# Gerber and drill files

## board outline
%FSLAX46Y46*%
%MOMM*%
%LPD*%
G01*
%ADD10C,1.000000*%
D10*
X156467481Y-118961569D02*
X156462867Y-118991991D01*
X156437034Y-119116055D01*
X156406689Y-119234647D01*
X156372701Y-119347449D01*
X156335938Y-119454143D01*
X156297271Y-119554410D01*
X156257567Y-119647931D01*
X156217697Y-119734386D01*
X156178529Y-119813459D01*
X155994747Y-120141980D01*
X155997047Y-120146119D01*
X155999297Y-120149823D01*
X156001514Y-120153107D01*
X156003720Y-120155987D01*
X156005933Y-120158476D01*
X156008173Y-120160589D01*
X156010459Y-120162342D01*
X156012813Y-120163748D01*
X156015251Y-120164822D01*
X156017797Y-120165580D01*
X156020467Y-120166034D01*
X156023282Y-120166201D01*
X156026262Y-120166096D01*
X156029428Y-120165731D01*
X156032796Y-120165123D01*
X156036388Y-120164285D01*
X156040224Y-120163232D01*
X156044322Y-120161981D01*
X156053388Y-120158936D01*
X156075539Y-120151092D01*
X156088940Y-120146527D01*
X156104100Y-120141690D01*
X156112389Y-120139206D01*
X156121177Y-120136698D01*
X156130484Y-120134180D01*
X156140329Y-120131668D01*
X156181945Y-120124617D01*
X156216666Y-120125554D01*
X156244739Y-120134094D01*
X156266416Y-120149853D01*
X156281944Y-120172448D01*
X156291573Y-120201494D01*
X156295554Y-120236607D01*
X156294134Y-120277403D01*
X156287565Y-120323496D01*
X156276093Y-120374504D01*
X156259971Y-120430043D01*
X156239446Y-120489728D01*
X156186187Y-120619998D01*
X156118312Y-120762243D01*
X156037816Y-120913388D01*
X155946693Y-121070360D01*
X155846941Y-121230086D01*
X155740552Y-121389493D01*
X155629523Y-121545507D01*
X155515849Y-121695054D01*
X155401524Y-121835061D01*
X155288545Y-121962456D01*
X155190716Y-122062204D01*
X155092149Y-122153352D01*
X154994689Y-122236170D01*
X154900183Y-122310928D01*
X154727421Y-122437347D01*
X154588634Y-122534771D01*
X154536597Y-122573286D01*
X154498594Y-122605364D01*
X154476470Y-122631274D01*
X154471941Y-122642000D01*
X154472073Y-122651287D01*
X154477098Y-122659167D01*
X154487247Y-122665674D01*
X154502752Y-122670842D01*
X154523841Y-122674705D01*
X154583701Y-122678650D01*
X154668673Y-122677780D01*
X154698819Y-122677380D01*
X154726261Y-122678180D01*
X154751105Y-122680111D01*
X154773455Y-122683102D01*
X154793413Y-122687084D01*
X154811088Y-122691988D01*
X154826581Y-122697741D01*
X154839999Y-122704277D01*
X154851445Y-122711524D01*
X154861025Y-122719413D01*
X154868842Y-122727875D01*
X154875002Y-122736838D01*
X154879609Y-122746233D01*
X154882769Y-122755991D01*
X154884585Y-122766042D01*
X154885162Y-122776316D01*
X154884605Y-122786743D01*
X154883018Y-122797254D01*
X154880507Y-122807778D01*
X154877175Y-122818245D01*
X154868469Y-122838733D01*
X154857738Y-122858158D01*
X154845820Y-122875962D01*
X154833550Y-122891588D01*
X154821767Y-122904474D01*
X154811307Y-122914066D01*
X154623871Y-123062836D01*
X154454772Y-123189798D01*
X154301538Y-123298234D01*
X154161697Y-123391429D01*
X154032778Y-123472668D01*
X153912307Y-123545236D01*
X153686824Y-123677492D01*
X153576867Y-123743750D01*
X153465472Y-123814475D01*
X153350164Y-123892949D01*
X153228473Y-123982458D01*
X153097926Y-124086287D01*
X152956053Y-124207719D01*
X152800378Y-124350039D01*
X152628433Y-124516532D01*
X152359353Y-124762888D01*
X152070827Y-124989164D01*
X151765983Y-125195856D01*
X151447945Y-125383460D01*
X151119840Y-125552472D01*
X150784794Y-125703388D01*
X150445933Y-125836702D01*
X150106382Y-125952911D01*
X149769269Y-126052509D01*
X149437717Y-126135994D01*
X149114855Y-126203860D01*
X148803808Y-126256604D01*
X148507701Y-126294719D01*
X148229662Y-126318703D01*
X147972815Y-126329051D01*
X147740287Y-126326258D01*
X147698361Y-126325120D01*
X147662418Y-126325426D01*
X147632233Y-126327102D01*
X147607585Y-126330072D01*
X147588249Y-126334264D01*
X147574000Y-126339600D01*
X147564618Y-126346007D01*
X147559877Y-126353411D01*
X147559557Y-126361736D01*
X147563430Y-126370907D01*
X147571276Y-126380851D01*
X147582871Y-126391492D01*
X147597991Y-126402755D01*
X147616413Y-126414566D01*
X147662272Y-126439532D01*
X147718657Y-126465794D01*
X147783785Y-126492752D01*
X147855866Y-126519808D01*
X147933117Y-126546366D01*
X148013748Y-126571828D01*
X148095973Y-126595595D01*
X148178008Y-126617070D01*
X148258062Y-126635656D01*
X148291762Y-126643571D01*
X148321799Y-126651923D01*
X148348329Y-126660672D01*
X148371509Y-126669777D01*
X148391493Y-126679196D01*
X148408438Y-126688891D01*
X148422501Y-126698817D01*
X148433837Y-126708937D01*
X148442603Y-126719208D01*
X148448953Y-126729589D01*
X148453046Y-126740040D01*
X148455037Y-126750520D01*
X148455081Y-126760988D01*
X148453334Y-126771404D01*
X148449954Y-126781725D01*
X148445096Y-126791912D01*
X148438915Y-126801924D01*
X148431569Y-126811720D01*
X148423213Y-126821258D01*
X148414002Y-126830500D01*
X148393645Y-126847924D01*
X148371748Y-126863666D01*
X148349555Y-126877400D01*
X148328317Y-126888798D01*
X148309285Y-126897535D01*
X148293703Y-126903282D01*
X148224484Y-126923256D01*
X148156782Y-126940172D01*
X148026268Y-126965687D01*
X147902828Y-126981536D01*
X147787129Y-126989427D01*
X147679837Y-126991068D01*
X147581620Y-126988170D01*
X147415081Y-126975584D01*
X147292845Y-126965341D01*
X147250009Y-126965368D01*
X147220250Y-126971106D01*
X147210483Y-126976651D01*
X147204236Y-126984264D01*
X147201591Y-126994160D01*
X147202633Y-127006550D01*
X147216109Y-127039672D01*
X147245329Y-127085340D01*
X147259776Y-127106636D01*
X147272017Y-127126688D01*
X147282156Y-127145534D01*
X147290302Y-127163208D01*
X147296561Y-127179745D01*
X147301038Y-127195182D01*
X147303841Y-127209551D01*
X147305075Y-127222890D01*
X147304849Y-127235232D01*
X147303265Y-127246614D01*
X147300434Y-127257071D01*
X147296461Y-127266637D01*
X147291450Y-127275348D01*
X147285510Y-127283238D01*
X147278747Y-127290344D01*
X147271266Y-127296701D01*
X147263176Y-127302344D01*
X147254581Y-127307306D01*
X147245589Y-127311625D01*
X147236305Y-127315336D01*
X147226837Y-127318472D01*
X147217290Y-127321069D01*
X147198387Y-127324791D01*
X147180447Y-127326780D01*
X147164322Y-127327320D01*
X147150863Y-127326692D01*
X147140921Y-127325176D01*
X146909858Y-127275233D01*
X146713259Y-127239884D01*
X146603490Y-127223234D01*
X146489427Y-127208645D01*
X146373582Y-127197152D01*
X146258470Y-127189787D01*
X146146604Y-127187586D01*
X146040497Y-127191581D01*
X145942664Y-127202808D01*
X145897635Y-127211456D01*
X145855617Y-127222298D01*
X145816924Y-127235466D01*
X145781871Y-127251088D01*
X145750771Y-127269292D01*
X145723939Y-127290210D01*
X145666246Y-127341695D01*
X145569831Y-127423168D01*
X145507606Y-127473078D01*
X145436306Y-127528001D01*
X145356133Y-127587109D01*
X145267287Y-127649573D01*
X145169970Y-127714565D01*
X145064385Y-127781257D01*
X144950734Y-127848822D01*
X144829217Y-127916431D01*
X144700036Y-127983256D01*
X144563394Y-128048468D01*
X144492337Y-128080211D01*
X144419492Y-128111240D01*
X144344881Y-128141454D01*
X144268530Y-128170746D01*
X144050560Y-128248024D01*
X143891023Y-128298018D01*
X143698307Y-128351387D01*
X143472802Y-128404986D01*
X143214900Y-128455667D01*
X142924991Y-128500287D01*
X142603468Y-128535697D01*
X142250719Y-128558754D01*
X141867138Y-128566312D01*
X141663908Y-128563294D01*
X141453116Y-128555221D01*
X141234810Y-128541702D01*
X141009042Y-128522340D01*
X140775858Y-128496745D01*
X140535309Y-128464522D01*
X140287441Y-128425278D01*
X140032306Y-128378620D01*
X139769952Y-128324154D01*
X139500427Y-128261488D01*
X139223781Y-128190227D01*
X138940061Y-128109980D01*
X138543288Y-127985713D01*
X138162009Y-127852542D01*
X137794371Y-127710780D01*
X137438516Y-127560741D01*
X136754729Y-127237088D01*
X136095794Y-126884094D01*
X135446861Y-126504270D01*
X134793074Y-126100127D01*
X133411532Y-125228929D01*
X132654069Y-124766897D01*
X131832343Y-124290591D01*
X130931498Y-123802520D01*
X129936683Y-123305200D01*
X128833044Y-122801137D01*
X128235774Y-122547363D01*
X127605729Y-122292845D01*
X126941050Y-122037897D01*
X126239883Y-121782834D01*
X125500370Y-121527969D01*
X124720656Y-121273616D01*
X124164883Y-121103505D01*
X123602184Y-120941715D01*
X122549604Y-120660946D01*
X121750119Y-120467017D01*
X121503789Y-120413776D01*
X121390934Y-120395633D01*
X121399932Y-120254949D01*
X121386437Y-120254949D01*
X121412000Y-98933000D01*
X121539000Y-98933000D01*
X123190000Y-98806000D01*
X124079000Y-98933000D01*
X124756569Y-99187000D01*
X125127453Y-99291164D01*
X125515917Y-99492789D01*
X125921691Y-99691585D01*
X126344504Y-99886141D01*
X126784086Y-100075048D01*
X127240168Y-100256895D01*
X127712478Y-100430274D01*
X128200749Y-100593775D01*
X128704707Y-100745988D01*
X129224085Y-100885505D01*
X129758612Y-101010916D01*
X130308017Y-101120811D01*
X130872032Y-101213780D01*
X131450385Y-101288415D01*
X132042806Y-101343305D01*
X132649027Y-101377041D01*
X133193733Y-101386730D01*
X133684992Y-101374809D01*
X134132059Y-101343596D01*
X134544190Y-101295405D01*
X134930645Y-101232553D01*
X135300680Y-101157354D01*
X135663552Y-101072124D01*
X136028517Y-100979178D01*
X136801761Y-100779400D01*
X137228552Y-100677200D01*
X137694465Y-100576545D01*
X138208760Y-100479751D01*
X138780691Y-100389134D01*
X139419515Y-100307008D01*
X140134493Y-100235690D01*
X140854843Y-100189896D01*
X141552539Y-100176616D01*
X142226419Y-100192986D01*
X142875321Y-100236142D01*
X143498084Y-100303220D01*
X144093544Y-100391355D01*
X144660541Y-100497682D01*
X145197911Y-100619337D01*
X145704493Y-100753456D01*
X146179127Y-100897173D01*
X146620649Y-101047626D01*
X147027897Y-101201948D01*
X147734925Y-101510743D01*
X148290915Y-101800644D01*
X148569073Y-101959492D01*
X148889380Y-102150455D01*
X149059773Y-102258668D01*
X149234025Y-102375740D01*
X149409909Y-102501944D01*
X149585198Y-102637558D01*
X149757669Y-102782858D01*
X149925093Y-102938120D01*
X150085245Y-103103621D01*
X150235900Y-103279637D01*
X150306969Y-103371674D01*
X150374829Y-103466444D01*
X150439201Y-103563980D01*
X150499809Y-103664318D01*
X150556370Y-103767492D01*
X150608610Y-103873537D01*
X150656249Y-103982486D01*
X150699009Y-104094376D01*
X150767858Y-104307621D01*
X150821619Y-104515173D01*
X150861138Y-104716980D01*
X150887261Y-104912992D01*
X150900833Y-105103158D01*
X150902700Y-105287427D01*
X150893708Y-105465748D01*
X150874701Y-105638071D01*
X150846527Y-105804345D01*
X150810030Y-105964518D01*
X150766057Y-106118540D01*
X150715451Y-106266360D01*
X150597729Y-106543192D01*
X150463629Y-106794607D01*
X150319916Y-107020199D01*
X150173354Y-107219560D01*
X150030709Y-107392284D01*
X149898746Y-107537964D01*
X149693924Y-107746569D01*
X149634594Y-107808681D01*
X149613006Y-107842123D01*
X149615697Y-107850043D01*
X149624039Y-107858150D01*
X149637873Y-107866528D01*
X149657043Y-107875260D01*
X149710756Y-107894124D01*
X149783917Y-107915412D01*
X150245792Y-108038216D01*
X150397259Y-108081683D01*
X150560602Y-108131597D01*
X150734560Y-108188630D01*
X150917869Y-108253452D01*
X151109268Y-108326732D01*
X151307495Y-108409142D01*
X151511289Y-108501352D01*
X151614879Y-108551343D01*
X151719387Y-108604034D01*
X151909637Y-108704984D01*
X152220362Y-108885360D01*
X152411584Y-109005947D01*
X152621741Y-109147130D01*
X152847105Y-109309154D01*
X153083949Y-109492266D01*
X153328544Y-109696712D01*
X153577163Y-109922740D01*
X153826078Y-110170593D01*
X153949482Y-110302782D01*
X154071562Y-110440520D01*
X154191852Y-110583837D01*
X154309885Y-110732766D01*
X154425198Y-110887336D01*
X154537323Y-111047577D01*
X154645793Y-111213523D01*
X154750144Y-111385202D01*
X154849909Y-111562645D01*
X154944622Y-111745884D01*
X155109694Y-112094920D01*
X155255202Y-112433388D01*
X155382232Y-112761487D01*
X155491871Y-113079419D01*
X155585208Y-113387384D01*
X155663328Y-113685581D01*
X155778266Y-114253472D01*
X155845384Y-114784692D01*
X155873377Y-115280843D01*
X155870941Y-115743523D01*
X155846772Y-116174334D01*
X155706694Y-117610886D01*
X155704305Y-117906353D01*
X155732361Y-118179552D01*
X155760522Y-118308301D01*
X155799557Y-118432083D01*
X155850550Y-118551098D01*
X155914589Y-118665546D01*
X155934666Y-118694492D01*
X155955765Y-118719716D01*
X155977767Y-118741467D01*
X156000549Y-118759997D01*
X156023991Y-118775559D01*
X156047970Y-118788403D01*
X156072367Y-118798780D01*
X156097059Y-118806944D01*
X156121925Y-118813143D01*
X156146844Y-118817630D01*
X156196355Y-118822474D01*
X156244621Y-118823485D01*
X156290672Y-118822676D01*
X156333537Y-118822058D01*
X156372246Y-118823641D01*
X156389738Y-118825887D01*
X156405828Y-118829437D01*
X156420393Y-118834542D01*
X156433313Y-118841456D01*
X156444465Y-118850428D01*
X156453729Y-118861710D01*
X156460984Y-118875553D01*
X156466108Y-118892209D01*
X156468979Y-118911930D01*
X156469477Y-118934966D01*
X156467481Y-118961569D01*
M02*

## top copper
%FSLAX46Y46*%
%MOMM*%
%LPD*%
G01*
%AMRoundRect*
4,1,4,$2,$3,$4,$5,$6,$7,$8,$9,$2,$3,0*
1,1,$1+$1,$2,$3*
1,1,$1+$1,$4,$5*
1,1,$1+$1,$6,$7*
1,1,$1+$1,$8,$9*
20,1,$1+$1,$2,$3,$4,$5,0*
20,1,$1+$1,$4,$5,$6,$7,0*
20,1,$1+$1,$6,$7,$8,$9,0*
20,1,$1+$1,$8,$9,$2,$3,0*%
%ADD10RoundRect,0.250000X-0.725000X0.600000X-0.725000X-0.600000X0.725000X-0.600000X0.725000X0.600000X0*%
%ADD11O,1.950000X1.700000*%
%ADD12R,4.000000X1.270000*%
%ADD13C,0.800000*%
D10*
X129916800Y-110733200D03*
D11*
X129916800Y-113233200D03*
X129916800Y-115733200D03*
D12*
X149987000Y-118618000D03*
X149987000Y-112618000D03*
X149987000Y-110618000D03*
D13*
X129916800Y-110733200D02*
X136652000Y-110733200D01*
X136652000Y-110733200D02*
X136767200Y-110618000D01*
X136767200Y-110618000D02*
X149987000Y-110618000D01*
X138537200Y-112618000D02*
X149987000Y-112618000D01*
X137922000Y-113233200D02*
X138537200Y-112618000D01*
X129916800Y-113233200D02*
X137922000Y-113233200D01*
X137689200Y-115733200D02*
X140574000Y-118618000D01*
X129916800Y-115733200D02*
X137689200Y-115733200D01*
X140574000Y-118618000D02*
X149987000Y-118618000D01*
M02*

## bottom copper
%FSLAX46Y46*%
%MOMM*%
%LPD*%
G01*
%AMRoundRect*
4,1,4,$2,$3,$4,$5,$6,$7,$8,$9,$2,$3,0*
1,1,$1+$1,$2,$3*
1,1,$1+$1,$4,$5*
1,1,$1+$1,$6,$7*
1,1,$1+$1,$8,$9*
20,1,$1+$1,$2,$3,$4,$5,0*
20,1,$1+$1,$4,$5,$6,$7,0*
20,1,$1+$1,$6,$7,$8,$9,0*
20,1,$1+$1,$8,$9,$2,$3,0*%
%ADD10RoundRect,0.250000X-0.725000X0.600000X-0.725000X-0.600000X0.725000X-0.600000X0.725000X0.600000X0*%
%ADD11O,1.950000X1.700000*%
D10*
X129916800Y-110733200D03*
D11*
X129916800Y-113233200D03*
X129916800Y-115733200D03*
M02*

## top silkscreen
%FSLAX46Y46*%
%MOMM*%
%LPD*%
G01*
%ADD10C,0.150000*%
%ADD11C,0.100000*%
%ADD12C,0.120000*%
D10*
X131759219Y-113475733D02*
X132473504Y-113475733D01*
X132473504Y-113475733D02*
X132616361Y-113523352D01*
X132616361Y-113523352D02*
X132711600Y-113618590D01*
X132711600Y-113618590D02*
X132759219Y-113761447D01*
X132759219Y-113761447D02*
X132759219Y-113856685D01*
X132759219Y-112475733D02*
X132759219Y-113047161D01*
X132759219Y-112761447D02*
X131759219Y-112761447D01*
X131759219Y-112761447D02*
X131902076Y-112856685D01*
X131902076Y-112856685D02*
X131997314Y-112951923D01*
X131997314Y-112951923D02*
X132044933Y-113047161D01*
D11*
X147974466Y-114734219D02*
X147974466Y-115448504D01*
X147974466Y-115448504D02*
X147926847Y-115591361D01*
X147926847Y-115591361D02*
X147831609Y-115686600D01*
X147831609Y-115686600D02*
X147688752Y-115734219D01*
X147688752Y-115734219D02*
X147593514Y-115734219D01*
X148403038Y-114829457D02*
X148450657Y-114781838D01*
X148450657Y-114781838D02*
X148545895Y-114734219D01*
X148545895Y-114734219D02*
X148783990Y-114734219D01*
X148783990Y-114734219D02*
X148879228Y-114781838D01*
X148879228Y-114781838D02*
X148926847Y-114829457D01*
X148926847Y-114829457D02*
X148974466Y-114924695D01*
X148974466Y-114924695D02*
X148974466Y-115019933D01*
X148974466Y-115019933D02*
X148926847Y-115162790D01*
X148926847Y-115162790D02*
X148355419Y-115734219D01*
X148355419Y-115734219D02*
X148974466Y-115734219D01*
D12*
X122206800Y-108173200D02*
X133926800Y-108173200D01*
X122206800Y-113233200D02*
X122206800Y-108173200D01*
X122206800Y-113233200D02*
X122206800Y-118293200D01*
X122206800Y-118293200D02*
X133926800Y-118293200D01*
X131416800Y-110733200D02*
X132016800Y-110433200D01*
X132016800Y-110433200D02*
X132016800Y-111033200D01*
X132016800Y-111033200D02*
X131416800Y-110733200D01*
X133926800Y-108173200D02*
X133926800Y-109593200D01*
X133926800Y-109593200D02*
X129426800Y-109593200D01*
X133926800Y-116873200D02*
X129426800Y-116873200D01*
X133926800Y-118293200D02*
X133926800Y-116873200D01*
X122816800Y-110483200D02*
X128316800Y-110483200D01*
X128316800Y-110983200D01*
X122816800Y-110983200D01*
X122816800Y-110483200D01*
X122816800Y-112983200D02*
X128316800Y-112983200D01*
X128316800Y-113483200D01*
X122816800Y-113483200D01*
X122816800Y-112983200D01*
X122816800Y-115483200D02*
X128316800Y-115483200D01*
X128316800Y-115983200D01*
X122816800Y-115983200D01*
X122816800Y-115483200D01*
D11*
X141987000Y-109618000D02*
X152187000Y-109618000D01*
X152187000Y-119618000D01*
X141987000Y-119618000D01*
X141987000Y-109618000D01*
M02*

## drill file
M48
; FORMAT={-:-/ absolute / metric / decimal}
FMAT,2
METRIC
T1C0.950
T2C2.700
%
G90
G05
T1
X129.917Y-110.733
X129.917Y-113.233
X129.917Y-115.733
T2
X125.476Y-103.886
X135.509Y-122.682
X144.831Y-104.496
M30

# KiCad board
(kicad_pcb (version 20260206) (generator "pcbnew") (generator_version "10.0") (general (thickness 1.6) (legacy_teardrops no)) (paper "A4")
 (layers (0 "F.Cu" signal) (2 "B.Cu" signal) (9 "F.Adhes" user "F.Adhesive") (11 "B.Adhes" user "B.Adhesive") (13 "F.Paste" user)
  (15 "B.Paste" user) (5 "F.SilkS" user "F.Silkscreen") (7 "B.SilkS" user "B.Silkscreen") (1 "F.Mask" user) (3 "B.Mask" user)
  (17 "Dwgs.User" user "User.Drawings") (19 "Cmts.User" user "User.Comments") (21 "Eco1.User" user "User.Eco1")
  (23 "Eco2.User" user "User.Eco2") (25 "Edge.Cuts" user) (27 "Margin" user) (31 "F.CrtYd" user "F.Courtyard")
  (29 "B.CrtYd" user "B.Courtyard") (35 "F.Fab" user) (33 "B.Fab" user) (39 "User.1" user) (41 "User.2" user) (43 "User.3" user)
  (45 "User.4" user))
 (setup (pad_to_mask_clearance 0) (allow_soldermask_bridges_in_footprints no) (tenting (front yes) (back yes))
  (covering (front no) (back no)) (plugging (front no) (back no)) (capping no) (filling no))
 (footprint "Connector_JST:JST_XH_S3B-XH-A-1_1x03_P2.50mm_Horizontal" (layer "F.Cu") (at 129.9168 110.7332 -90)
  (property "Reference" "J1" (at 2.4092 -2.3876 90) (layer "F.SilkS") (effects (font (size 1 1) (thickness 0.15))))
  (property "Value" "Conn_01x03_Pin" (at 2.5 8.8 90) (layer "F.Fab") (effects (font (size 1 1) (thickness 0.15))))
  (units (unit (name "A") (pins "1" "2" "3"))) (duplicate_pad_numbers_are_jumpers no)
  (fp_line (start -2.56 7.71) (end -2.56 -4.01) (stroke (width 0.12) (type solid)) (layer "F.SilkS"))
  (fp_line (start 2.5 7.71) (end -2.56 7.71) (stroke (width 0.12) (type solid)) (layer "F.SilkS"))
  (fp_line (start 2.5 7.71) (end 7.56 7.71) (stroke (width 0.12) (type solid)) (layer "F.SilkS"))
  (fp_line (start 7.56 7.71) (end 7.56 -4.01) (stroke (width 0.12) (type solid)) (layer "F.SilkS"))
  (fp_line (start 0 -1.5) (end -0.3 -2.1) (stroke (width 0.12) (type solid)) (layer "F.SilkS"))
  (fp_line (start -0.3 -2.1) (end 0.3 -2.1) (stroke (width 0.12) (type solid)) (layer "F.SilkS"))
  (fp_line (start 0.3 -2.1) (end 0 -1.5) (stroke (width 0.12) (type solid)) (layer "F.SilkS"))
  (fp_line (start -2.56 -4.01) (end -1.14 -4.01) (stroke (width 0.12) (type solid)) (layer "F.SilkS"))
  (fp_line (start -1.14 -4.01) (end -1.14 0.49) (stroke (width 0.12) (type solid)) (layer "F.SilkS"))
  (fp_line (start 6.14 -4.01) (end 6.14 0.49) (stroke (width 0.12) (type solid)) (layer "F.SilkS"))
  (fp_line (start 7.56 -4.01) (end 6.14 -4.01) (stroke (width 0.12) (type solid)) (layer "F.SilkS"))
  (fp_rect (start -0.25 1.6) (end 0.25 7.1) (stroke (width 0.12) (type solid)) (fill no) (layer "F.SilkS"))
  (fp_rect (start 2.25 1.6) (end 2.75 7.1) (stroke (width 0.12) (type solid)) (fill no) (layer "F.SilkS"))
  (fp_rect (start 4.75 1.6) (end 5.25 7.1) (stroke (width 0.12) (type solid)) (fill no) (layer "F.SilkS"))
  (pad "1" thru_hole roundrect (at 0 0 270) (size 1.7 1.95) (drill 0.95) (layers "*.Cu" "*.Mask") (remove_unused_layers no)
   (roundrect_rratio 0.147059) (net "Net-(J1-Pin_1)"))
  (pad "2" thru_hole oval (at 2.5 0 270) (size 1.7 1.95) (drill 0.95) (layers "*.Cu" "*.Mask") (remove_unused_layers no)
   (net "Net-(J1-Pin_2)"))
  (pad "3" thru_hole oval (at 5 0 270) (size 1.7 1.95) (drill 0.95) (layers "*.Cu" "*.Mask") (remove_unused_layers no)
   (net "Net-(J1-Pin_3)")))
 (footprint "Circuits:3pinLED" (layer "F.Cu") (at 144.987 119.618)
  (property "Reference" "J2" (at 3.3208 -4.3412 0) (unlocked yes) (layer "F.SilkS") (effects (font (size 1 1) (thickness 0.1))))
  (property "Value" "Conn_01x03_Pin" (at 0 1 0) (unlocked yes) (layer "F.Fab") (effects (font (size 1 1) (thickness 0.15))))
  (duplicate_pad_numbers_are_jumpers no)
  (fp_rect (start -3 -10) (end 7.2 0) (stroke (width 0.1) (type solid)) (fill no) (layer "F.SilkS"))
  (pad "1" smd rect (at 5 -1 180) (size 4 1.27) (layers "F.Cu" "F.Mask" "F.Paste") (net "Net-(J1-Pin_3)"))
  (pad "2" smd rect (at 5 -7 180) (size 4 1.27) (layers "F.Cu" "F.Mask" "F.Paste") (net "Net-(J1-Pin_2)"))
  (pad "3" smd rect (at 5 -9 180) (size 4 1.27) (layers "F.Cu" "F.Mask" "F.Paste") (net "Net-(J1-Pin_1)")))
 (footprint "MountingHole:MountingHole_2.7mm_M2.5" (layer "F.Cu") (at 144.8308 104.4956)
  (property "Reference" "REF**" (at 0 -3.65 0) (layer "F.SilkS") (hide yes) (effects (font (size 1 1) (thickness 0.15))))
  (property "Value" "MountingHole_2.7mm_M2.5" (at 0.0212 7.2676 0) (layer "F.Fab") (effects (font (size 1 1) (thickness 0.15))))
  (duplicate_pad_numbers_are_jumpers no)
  (pad "" np_thru_hole circle (at 0 0) (size 2.7 2.7) (drill 2.7) (layers "*.Cu" "*.Mask")))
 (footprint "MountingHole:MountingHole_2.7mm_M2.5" (layer "F.Cu") (at 125.476 103.886)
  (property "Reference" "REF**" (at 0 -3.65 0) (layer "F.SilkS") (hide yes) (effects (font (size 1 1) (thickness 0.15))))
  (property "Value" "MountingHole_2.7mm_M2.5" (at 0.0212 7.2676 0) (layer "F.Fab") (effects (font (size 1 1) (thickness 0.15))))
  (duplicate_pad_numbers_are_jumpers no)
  (pad "" np_thru_hole circle (at 0 0) (size 2.7 2.7) (drill 2.7) (layers "*.Cu" "*.Mask")))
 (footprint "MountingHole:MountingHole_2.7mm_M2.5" (layer "F.Cu") (at 135.509 122.682)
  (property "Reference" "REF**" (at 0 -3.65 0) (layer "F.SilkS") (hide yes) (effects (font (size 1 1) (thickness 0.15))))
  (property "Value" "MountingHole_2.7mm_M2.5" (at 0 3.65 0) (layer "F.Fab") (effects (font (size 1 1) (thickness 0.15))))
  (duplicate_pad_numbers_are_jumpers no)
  (pad "" np_thru_hole circle (at 0 0) (size 2.7 2.7) (drill 2.7) (layers "*.Cu" "*.Mask")))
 (gr_poly
  (pts (xy 156.467481 118.961569) (xy 156.462867 118.991991) (xy 156.437034 119.116055) (xy 156.406689 119.234647)
   (xy 156.372701 119.347449) (xy 156.335938 119.454143) (xy 156.297271 119.55441) (xy 156.257567 119.647931) (xy 156.217697 119.734386)
   (xy 156.178529 119.813459) (xy 155.994747 120.14198) (xy 155.997047 120.146119) (xy 155.999297 120.149823) (xy 156.001514 120.153107)
   (xy 156.00372 120.155987) (xy 156.005933 120.158476) (xy 156.008173 120.160589) (xy 156.010459 120.162342) (xy 156.012813 120.163748)
   (xy 156.015251 120.164822) (xy 156.017797 120.16558) (xy 156.020467 120.166034) (xy 156.023282 120.166201) (xy 156.026262 120.166096)
   (xy 156.029428 120.165731) (xy 156.032796 120.165123) (xy 156.036388 120.164285) (xy 156.040224 120.163232) (xy 156.044322 120.161981)
   (xy 156.053388 120.158936) (xy 156.075539 120.151092) (xy 156.08894 120.146527) (xy 156.1041 120.14169) (xy 156.112389 120.139206)
   (xy 156.121177 120.136698) (xy 156.130484 120.13418) (xy 156.140329 120.131668) (xy 156.181945 120.124617) (xy 156.216666 120.125554)
   (xy 156.244739 120.134094) (xy 156.266416 120.149853) (xy 156.281944 120.172448) (xy 156.291573 120.201494) (xy 156.295554 120.236607)
   (xy 156.294134 120.277403) (xy 156.287565 120.323496) (xy 156.276093 120.374504) (xy 156.259971 120.430043) (xy 156.239446 120.489728)
   (xy 156.186187 120.619998) (xy 156.118312 120.762243) (xy 156.037816 120.913388) (xy 155.946693 121.07036) (xy 155.846941 121.230086)
   (xy 155.740552 121.389493) (xy 155.629523 121.545507) (xy 155.515849 121.695054) (xy 155.401524 121.835061) (xy 155.288545 121.962456)
   (xy 155.190716 122.062204) (xy 155.092149 122.153352) (xy 154.994689 122.23617) (xy 154.900183 122.310928) (xy 154.727421 122.437347)
   (xy 154.588634 122.534771) (xy 154.536597 122.573286) (xy 154.498594 122.605364) (xy 154.47647 122.631274) (xy 154.471941 122.642)
   (xy 154.472073 122.651287) (xy 154.477098 122.659167) (xy 154.487247 122.665674) (xy 154.502752 122.670842) (xy 154.523841 122.674705)
   (xy 154.583701 122.67865) (xy 154.668673 122.67778) (xy 154.698819 122.67738) (xy 154.726261 122.67818) (xy 154.751105 122.680111)
   (xy 154.773455 122.683102) (xy 154.793413 122.687084) (xy 154.811088 122.691988) (xy 154.826581 122.697741) (xy 154.839999 122.704277)
   (xy 154.851445 122.711524) (xy 154.861025 122.719413) (xy 154.868842 122.727875) (xy 154.875002 122.736838) (xy 154.879609 122.746233)
   (xy 154.882769 122.755991) (xy 154.884585 122.766042) (xy 154.885162 122.776316) (xy 154.884605 122.786743) (xy 154.883018 122.797254)
   (xy 154.880507 122.807778) (xy 154.877175 122.818245) (xy 154.868469 122.838733) (xy 154.857738 122.858158) (xy 154.84582 122.875962)
   (xy 154.83355 122.891588) (xy 154.821767 122.904474) (xy 154.811307 122.914066) (xy 154.623871 123.062836) (xy 154.454772 123.189798)
   (xy 154.301538 123.298234) (xy 154.161697 123.391429) (xy 154.032778 123.472668) (xy 153.912307 123.545236) (xy 153.686824 123.677492)
   (xy 153.576867 123.74375) (xy 153.465472 123.814475) (xy 153.350164 123.892949) (xy 153.228473 123.982458) (xy 153.097926 124.086287)
   (xy 152.956053 124.207719) (xy 152.800378 124.350039) (xy 152.628433 124.516532) (xy 152.359353 124.762888) (xy 152.070827 124.989164)
   (xy 151.765983 125.195856) (xy 151.447945 125.38346) (xy 151.11984 125.552472) (xy 150.784794 125.703388) (xy 150.445933 125.836702)
   (xy 150.106382 125.952911) (xy 149.769269 126.052509) (xy 149.437717 126.135994) (xy 149.114855 126.20386) (xy 148.803808 126.256604)
   (xy 148.507701 126.294719) (xy 148.229662 126.318703) (xy 147.972815 126.329051) (xy 147.740287 126.326258) (xy 147.698361 126.32512)
   (xy 147.662418 126.325426) (xy 147.632233 126.327102) (xy 147.607585 126.330072) (xy 147.588249 126.334264) (xy 147.574 126.3396)
   (xy 147.564618 126.346007) (xy 147.559877 126.353411) (xy 147.559557 126.361736) (xy 147.56343 126.370907) (xy 147.571276 126.380851)
   (xy 147.582871 126.391492) (xy 147.597991 126.402755) (xy 147.616413 126.414566) (xy 147.662272 126.439532) (xy 147.718657 126.465794)
   (xy 147.783785 126.492752) (xy 147.855866 126.519808) (xy 147.933117 126.546366) (xy 148.013748 126.571828) (xy 148.095973 126.595595)
   (xy 148.178008 126.61707) (xy 148.258062 126.635656) (xy 148.291762 126.643571) (xy 148.321799 126.651923) (xy 148.348329 126.660672)
   (xy 148.371509 126.669777) (xy 148.391493 126.679196) (xy 148.408438 126.688891) (xy 148.422501 126.698817) (xy 148.433837 126.708937)
   (xy 148.442603 126.719208) (xy 148.448953 126.729589) (xy 148.453046 126.74004) (xy 148.455037 126.75052) (xy 148.455081 126.760988)
   (xy 148.453334 126.771404) (xy 148.449954 126.781725) (xy 148.445096 126.791912) (xy 148.438915 126.801924) (xy 148.431569 126.81172)
   (xy 148.423213 126.821258) (xy 148.414002 126.8305) (xy 148.393645 126.847924) (xy 148.371748 126.863666) (xy 148.349555 126.8774)
   (xy 148.328317 126.888798) (xy 148.309285 126.897535) (xy 148.293703 126.903282) (xy 148.224484 126.923256) (xy 148.156782 126.940172)
   (xy 148.026268 126.965687) (xy 147.902828 126.981536) (xy 147.787129 126.989427) (xy 147.679837 126.991068) (xy 147.58162 126.98817)
   (xy 147.415081 126.975584) (xy 147.292845 126.965341) (xy 147.250009 126.965368) (xy 147.22025 126.971106) (xy 147.210483 126.976651)
   (xy 147.204236 126.984264) (xy 147.201591 126.99416) (xy 147.202633 127.00655) (xy 147.216109 127.039672) (xy 147.245329 127.08534)
   (xy 147.259776 127.106636) (xy 147.272017 127.126688) (xy 147.282156 127.145534) (xy 147.290302 127.163208) (xy 147.296561 127.179745)
   (xy 147.301038 127.195182) (xy 147.303841 127.209551) (xy 147.305075 127.22289) (xy 147.304849 127.235232) (xy 147.303265 127.246614)
   (xy 147.300434 127.257071) (xy 147.296461 127.266637) (xy 147.29145 127.275348) (xy 147.28551 127.283238) (xy 147.278747 127.290344)
   (xy 147.271266 127.296701) (xy 147.263176 127.302344) (xy 147.254581 127.307306) (xy 147.245589 127.311625) (xy 147.236305 127.315336)
   (xy 147.226837 127.318472) (xy 147.21729 127.321069) (xy 147.198387 127.324791) (xy 147.180447 127.32678) (xy 147.164322 127.32732)
   (xy 147.150863 127.326692) (xy 147.140921 127.325176) (xy 146.909858 127.275233) (xy 146.713259 127.239884) (xy 146.60349 127.223234)
   (xy 146.489427 127.208645) (xy 146.373582 127.197152) (xy 146.25847 127.189787) (xy 146.146604 127.187586) (xy 146.040497 127.191581)
   (xy 145.942664 127.202808) (xy 145.897635 127.211456) (xy 145.855617 127.222298) (xy 145.816924 127.235466) (xy 145.781871 127.251088)
   (xy 145.750771 127.269292) (xy 145.723939 127.29021) (xy 145.666246 127.341695) (xy 145.569831 127.423168) (xy 145.507606 127.473078)
   (xy 145.436306 127.528001) (xy 145.356133 127.587109) (xy 145.267287 127.649573) (xy 145.16997 127.714565) (xy 145.064385 127.781257)
   (xy 144.950734 127.848822) (xy 144.829217 127.916431) (xy 144.700036 127.983256) (xy 144.563394 128.048468) (xy 144.492337 128.080211)
   (xy 144.419492 128.11124) (xy 144.344881 128.141454) (xy 144.26853 128.170746) (xy 144.05056 128.248024) (xy 143.891023 128.298018)
   (xy 143.698307 128.351387) (xy 143.472802 128.404986) (xy 143.2149 128.455667) (xy 142.924991 128.500287) (xy 142.603468 128.535697)
   (xy 142.250719 128.558754) (xy 141.867138 128.566312) (xy 141.663908 128.563294) (xy 141.453116 128.555221) (xy 141.23481 128.541702)
   (xy 141.009042 128.52234) (xy 140.775858 128.496745) (xy 140.535309 128.464522) (xy 140.287441 128.425278) (xy 140.032306 128.37862)
   (xy 139.769952 128.324154) (xy 139.500427 128.261488) (xy 139.223781 128.190227) (xy 138.940061 128.10998) (xy 138.543288 127.985713)
   (xy 138.162009 127.852542) (xy 137.794371 127.71078) (xy 137.438516 127.560741) (xy 136.754729 127.237088) (xy 136.095794 126.884094)
   (xy 135.446861 126.50427) (xy 134.793074 126.100127) (xy 133.411532 125.228929) (xy 132.654069 124.766897) (xy 131.832343 124.290591)
   (xy 130.931498 123.80252) (xy 129.936683 123.3052) (xy 128.833044 122.801137) (xy 128.235774 122.547363) (xy 127.605729 122.292845)
   (xy 126.94105 122.037897) (xy 126.239883 121.782834) (xy 125.50037 121.527969) (xy 124.720656 121.273616) (xy 124.164883 121.103505)
   (xy 123.602184 120.941715) (xy 122.549604 120.660946) (xy 121.750119 120.467017) (xy 121.503789 120.413776) (xy 121.390934 120.395633)
   (xy 121.399932 120.254949) (xy 121.386437 120.254949) (xy 121.412 98.933) (xy 121.539 98.933) (xy 123.19 98.806) (xy 124.079 98.933)
   (xy 124.756569 99.187) (xy 125.127453 99.291164) (xy 125.515917 99.492789) (xy 125.921691 99.691585) (xy 126.344504 99.886141)
   (xy 126.784086 100.075048) (xy 127.240168 100.256895) (xy 127.712478 100.430274) (xy 128.200749 100.593775) (xy 128.704707 100.745988)
   (xy 129.224085 100.885505) (xy 129.758612 101.010916) (xy 130.308017 101.120811) (xy 130.872032 101.21378) (xy 131.450385 101.288415)
   (xy 132.042806 101.343305) (xy 132.649027 101.377041) (xy 133.193733 101.38673) (xy 133.684992 101.374809) (xy 134.132059 101.343596)
   (xy 134.54419 101.295405) (xy 134.930645 101.232553) (xy 135.30068 101.157354) (xy 135.663552 101.072124) (xy 136.028517 100.979178)
   (xy 136.801761 100.7794) (xy 137.228552 100.6772) (xy 137.694465 100.576545) (xy 138.20876 100.479751) (xy 138.780691 100.389134)
   (xy 139.419515 100.307008) (xy 140.134493 100.23569) (xy 140.854843 100.189896) (xy 141.552539 100.176616) (xy 142.226419 100.192986)
   (xy 142.875321 100.236142) (xy 143.498084 100.30322) (xy 144.093544 100.391355) (xy 144.660541 100.497682) (xy 145.197911 100.619337)
   (xy 145.704493 100.753456) (xy 146.179127 100.897173) (xy 146.620649 101.047626) (xy 147.027897 101.201948) (xy 147.734925 101.510743)
   (xy 148.290915 101.800644) (xy 148.569073 101.959492) (xy 148.88938 102.150455) (xy 149.059773 102.258668) (xy 149.234025 102.37574)
   (xy 149.409909 102.501944) (xy 149.585198 102.637558) (xy 149.757669 102.782858) (xy 149.925093 102.93812) (xy 150.085245 103.103621)
   (xy 150.2359 103.279637) (xy 150.306969 103.371674) (xy 150.374829 103.466444) (xy 150.439201 103.56398) (xy 150.499809 103.664318)
   (xy 150.55637 103.767492) (xy 150.60861 103.873537) (xy 150.656249 103.982486) (xy 150.699009 104.094376) (xy 150.767858 104.307621)
   (xy 150.821619 104.515173) (xy 150.861138 104.71698) (xy 150.887261 104.912992) (xy 150.900833 105.103158) (xy 150.9027 105.287427)
   (xy 150.893708 105.465748) (xy 150.874701 105.638071) (xy 150.846527 105.804345) (xy 150.81003 105.964518) (xy 150.766057 106.11854)
   (xy 150.715451 106.26636) (xy 150.597729 106.543192) (xy 150.463629 106.794607) (xy 150.319916 107.020199) (xy 150.173354 107.21956)
   (xy 150.030709 107.392284) (xy 149.898746 107.537964) (xy 149.693924 107.746569) (xy 149.634594 107.808681) (xy 149.613006 107.842123)
   (xy 149.615697 107.850043) (xy 149.624039 107.85815) (xy 149.637873 107.866528) (xy 149.657043 107.87526) (xy 149.710756 107.894124)
   (xy 149.783917 107.915412) (xy 150.245792 108.038216) (xy 150.397259 108.081683) (xy 150.560602 108.131597) (xy 150.73456 108.18863)
   (xy 150.917869 108.253452) (xy 151.109268 108.326732) (xy 151.307495 108.409142) (xy 151.511289 108.501352) (xy 151.614879 108.551343)
   (xy 151.719387 108.604034) (xy 151.909637 108.704984) (xy 152.220362 108.88536) (xy 152.411584 109.005947) (xy 152.621741 109.14713)
   (xy 152.847105 109.309154) (xy 153.083949 109.492266) (xy 153.328544 109.696712) (xy 153.577163 109.92274) (xy 153.826078 110.170593)
   (xy 153.949482 110.302782) (xy 154.071562 110.44052) (xy 154.191852 110.583837) (xy 154.309885 110.732766) (xy 154.425198 110.887336)
   (xy 154.537323 111.047577) (xy 154.645793 111.213523) (xy 154.750144 111.385202) (xy 154.849909 111.562645) (xy 154.944622 111.745884)
   (xy 155.109694 112.09492) (xy 155.255202 112.433388) (xy 155.382232 112.761487) (xy 155.491871 113.079419) (xy 155.585208 113.387384)
   (xy 155.663328 113.685581) (xy 155.778266 114.253472) (xy 155.845384 114.784692) (xy 155.873377 115.280843) (xy 155.870941 115.743523)
   (xy 155.846772 116.174334) (xy 155.706694 117.610886) (xy 155.704305 117.906353) (xy 155.732361 118.179552) (xy 155.760522 118.308301)
   (xy 155.799557 118.432083) (xy 155.85055 118.551098) (xy 155.914589 118.665546) (xy 155.934666 118.694492) (xy 155.955765 118.719716)
   (xy 155.977767 118.741467) (xy 156.000549 118.759997) (xy 156.023991 118.775559) (xy 156.04797 118.788403) (xy 156.072367 118.79878)
   (xy 156.097059 118.806944) (xy 156.121925 118.813143) (xy 156.146844 118.81763) (xy 156.196355 118.822474) (xy 156.244621 118.823485)
   (xy 156.290672 118.822676) (xy 156.333537 118.822058) (xy 156.372246 118.823641) (xy 156.389738 118.825887) (xy 156.405828 118.829437)
   (xy 156.420393 118.834542) (xy 156.433313 118.841456) (xy 156.444465 118.850428) (xy 156.453729 118.86171) (xy 156.460984 118.875553)
   (xy 156.466108 118.892209) (xy 156.468979 118.91193) (xy 156.469477 118.934966))
  (stroke (width 1) (type solid)) (fill no) (layer "Edge.Cuts"))
 (segment (start 129.9168 110.7332) (end 136.652 110.7332) (width 0.8) (layer "F.Cu") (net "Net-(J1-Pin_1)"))
 (segment (start 136.652 110.7332) (end 136.7672 110.618) (width 0.8) (layer "F.Cu") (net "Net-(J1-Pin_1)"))
 (segment (start 136.7672 110.618) (end 149.987 110.618) (width 0.8) (layer "F.Cu") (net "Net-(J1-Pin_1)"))
 (segment (start 138.5372 112.618) (end 149.987 112.618) (width 0.8) (layer "F.Cu") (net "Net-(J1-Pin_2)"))
 (segment (start 137.922 113.2332) (end 138.5372 112.618) (width 0.8) (layer "F.Cu") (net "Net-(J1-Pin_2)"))
 (segment (start 129.9168 113.2332) (end 137.922 113.2332) (width 0.8) (layer "F.Cu") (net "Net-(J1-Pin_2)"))
 (segment (start 137.6892 115.7332) (end 140.574 118.618) (width 0.8) (layer "F.Cu") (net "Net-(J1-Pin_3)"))
 (segment (start 129.9168 115.7332) (end 137.6892 115.7332) (width 0.8) (layer "F.Cu") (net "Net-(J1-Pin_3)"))
 (segment (start 140.574 118.618) (end 149.987 118.618) (width 0.8) (layer "F.Cu") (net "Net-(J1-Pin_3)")))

